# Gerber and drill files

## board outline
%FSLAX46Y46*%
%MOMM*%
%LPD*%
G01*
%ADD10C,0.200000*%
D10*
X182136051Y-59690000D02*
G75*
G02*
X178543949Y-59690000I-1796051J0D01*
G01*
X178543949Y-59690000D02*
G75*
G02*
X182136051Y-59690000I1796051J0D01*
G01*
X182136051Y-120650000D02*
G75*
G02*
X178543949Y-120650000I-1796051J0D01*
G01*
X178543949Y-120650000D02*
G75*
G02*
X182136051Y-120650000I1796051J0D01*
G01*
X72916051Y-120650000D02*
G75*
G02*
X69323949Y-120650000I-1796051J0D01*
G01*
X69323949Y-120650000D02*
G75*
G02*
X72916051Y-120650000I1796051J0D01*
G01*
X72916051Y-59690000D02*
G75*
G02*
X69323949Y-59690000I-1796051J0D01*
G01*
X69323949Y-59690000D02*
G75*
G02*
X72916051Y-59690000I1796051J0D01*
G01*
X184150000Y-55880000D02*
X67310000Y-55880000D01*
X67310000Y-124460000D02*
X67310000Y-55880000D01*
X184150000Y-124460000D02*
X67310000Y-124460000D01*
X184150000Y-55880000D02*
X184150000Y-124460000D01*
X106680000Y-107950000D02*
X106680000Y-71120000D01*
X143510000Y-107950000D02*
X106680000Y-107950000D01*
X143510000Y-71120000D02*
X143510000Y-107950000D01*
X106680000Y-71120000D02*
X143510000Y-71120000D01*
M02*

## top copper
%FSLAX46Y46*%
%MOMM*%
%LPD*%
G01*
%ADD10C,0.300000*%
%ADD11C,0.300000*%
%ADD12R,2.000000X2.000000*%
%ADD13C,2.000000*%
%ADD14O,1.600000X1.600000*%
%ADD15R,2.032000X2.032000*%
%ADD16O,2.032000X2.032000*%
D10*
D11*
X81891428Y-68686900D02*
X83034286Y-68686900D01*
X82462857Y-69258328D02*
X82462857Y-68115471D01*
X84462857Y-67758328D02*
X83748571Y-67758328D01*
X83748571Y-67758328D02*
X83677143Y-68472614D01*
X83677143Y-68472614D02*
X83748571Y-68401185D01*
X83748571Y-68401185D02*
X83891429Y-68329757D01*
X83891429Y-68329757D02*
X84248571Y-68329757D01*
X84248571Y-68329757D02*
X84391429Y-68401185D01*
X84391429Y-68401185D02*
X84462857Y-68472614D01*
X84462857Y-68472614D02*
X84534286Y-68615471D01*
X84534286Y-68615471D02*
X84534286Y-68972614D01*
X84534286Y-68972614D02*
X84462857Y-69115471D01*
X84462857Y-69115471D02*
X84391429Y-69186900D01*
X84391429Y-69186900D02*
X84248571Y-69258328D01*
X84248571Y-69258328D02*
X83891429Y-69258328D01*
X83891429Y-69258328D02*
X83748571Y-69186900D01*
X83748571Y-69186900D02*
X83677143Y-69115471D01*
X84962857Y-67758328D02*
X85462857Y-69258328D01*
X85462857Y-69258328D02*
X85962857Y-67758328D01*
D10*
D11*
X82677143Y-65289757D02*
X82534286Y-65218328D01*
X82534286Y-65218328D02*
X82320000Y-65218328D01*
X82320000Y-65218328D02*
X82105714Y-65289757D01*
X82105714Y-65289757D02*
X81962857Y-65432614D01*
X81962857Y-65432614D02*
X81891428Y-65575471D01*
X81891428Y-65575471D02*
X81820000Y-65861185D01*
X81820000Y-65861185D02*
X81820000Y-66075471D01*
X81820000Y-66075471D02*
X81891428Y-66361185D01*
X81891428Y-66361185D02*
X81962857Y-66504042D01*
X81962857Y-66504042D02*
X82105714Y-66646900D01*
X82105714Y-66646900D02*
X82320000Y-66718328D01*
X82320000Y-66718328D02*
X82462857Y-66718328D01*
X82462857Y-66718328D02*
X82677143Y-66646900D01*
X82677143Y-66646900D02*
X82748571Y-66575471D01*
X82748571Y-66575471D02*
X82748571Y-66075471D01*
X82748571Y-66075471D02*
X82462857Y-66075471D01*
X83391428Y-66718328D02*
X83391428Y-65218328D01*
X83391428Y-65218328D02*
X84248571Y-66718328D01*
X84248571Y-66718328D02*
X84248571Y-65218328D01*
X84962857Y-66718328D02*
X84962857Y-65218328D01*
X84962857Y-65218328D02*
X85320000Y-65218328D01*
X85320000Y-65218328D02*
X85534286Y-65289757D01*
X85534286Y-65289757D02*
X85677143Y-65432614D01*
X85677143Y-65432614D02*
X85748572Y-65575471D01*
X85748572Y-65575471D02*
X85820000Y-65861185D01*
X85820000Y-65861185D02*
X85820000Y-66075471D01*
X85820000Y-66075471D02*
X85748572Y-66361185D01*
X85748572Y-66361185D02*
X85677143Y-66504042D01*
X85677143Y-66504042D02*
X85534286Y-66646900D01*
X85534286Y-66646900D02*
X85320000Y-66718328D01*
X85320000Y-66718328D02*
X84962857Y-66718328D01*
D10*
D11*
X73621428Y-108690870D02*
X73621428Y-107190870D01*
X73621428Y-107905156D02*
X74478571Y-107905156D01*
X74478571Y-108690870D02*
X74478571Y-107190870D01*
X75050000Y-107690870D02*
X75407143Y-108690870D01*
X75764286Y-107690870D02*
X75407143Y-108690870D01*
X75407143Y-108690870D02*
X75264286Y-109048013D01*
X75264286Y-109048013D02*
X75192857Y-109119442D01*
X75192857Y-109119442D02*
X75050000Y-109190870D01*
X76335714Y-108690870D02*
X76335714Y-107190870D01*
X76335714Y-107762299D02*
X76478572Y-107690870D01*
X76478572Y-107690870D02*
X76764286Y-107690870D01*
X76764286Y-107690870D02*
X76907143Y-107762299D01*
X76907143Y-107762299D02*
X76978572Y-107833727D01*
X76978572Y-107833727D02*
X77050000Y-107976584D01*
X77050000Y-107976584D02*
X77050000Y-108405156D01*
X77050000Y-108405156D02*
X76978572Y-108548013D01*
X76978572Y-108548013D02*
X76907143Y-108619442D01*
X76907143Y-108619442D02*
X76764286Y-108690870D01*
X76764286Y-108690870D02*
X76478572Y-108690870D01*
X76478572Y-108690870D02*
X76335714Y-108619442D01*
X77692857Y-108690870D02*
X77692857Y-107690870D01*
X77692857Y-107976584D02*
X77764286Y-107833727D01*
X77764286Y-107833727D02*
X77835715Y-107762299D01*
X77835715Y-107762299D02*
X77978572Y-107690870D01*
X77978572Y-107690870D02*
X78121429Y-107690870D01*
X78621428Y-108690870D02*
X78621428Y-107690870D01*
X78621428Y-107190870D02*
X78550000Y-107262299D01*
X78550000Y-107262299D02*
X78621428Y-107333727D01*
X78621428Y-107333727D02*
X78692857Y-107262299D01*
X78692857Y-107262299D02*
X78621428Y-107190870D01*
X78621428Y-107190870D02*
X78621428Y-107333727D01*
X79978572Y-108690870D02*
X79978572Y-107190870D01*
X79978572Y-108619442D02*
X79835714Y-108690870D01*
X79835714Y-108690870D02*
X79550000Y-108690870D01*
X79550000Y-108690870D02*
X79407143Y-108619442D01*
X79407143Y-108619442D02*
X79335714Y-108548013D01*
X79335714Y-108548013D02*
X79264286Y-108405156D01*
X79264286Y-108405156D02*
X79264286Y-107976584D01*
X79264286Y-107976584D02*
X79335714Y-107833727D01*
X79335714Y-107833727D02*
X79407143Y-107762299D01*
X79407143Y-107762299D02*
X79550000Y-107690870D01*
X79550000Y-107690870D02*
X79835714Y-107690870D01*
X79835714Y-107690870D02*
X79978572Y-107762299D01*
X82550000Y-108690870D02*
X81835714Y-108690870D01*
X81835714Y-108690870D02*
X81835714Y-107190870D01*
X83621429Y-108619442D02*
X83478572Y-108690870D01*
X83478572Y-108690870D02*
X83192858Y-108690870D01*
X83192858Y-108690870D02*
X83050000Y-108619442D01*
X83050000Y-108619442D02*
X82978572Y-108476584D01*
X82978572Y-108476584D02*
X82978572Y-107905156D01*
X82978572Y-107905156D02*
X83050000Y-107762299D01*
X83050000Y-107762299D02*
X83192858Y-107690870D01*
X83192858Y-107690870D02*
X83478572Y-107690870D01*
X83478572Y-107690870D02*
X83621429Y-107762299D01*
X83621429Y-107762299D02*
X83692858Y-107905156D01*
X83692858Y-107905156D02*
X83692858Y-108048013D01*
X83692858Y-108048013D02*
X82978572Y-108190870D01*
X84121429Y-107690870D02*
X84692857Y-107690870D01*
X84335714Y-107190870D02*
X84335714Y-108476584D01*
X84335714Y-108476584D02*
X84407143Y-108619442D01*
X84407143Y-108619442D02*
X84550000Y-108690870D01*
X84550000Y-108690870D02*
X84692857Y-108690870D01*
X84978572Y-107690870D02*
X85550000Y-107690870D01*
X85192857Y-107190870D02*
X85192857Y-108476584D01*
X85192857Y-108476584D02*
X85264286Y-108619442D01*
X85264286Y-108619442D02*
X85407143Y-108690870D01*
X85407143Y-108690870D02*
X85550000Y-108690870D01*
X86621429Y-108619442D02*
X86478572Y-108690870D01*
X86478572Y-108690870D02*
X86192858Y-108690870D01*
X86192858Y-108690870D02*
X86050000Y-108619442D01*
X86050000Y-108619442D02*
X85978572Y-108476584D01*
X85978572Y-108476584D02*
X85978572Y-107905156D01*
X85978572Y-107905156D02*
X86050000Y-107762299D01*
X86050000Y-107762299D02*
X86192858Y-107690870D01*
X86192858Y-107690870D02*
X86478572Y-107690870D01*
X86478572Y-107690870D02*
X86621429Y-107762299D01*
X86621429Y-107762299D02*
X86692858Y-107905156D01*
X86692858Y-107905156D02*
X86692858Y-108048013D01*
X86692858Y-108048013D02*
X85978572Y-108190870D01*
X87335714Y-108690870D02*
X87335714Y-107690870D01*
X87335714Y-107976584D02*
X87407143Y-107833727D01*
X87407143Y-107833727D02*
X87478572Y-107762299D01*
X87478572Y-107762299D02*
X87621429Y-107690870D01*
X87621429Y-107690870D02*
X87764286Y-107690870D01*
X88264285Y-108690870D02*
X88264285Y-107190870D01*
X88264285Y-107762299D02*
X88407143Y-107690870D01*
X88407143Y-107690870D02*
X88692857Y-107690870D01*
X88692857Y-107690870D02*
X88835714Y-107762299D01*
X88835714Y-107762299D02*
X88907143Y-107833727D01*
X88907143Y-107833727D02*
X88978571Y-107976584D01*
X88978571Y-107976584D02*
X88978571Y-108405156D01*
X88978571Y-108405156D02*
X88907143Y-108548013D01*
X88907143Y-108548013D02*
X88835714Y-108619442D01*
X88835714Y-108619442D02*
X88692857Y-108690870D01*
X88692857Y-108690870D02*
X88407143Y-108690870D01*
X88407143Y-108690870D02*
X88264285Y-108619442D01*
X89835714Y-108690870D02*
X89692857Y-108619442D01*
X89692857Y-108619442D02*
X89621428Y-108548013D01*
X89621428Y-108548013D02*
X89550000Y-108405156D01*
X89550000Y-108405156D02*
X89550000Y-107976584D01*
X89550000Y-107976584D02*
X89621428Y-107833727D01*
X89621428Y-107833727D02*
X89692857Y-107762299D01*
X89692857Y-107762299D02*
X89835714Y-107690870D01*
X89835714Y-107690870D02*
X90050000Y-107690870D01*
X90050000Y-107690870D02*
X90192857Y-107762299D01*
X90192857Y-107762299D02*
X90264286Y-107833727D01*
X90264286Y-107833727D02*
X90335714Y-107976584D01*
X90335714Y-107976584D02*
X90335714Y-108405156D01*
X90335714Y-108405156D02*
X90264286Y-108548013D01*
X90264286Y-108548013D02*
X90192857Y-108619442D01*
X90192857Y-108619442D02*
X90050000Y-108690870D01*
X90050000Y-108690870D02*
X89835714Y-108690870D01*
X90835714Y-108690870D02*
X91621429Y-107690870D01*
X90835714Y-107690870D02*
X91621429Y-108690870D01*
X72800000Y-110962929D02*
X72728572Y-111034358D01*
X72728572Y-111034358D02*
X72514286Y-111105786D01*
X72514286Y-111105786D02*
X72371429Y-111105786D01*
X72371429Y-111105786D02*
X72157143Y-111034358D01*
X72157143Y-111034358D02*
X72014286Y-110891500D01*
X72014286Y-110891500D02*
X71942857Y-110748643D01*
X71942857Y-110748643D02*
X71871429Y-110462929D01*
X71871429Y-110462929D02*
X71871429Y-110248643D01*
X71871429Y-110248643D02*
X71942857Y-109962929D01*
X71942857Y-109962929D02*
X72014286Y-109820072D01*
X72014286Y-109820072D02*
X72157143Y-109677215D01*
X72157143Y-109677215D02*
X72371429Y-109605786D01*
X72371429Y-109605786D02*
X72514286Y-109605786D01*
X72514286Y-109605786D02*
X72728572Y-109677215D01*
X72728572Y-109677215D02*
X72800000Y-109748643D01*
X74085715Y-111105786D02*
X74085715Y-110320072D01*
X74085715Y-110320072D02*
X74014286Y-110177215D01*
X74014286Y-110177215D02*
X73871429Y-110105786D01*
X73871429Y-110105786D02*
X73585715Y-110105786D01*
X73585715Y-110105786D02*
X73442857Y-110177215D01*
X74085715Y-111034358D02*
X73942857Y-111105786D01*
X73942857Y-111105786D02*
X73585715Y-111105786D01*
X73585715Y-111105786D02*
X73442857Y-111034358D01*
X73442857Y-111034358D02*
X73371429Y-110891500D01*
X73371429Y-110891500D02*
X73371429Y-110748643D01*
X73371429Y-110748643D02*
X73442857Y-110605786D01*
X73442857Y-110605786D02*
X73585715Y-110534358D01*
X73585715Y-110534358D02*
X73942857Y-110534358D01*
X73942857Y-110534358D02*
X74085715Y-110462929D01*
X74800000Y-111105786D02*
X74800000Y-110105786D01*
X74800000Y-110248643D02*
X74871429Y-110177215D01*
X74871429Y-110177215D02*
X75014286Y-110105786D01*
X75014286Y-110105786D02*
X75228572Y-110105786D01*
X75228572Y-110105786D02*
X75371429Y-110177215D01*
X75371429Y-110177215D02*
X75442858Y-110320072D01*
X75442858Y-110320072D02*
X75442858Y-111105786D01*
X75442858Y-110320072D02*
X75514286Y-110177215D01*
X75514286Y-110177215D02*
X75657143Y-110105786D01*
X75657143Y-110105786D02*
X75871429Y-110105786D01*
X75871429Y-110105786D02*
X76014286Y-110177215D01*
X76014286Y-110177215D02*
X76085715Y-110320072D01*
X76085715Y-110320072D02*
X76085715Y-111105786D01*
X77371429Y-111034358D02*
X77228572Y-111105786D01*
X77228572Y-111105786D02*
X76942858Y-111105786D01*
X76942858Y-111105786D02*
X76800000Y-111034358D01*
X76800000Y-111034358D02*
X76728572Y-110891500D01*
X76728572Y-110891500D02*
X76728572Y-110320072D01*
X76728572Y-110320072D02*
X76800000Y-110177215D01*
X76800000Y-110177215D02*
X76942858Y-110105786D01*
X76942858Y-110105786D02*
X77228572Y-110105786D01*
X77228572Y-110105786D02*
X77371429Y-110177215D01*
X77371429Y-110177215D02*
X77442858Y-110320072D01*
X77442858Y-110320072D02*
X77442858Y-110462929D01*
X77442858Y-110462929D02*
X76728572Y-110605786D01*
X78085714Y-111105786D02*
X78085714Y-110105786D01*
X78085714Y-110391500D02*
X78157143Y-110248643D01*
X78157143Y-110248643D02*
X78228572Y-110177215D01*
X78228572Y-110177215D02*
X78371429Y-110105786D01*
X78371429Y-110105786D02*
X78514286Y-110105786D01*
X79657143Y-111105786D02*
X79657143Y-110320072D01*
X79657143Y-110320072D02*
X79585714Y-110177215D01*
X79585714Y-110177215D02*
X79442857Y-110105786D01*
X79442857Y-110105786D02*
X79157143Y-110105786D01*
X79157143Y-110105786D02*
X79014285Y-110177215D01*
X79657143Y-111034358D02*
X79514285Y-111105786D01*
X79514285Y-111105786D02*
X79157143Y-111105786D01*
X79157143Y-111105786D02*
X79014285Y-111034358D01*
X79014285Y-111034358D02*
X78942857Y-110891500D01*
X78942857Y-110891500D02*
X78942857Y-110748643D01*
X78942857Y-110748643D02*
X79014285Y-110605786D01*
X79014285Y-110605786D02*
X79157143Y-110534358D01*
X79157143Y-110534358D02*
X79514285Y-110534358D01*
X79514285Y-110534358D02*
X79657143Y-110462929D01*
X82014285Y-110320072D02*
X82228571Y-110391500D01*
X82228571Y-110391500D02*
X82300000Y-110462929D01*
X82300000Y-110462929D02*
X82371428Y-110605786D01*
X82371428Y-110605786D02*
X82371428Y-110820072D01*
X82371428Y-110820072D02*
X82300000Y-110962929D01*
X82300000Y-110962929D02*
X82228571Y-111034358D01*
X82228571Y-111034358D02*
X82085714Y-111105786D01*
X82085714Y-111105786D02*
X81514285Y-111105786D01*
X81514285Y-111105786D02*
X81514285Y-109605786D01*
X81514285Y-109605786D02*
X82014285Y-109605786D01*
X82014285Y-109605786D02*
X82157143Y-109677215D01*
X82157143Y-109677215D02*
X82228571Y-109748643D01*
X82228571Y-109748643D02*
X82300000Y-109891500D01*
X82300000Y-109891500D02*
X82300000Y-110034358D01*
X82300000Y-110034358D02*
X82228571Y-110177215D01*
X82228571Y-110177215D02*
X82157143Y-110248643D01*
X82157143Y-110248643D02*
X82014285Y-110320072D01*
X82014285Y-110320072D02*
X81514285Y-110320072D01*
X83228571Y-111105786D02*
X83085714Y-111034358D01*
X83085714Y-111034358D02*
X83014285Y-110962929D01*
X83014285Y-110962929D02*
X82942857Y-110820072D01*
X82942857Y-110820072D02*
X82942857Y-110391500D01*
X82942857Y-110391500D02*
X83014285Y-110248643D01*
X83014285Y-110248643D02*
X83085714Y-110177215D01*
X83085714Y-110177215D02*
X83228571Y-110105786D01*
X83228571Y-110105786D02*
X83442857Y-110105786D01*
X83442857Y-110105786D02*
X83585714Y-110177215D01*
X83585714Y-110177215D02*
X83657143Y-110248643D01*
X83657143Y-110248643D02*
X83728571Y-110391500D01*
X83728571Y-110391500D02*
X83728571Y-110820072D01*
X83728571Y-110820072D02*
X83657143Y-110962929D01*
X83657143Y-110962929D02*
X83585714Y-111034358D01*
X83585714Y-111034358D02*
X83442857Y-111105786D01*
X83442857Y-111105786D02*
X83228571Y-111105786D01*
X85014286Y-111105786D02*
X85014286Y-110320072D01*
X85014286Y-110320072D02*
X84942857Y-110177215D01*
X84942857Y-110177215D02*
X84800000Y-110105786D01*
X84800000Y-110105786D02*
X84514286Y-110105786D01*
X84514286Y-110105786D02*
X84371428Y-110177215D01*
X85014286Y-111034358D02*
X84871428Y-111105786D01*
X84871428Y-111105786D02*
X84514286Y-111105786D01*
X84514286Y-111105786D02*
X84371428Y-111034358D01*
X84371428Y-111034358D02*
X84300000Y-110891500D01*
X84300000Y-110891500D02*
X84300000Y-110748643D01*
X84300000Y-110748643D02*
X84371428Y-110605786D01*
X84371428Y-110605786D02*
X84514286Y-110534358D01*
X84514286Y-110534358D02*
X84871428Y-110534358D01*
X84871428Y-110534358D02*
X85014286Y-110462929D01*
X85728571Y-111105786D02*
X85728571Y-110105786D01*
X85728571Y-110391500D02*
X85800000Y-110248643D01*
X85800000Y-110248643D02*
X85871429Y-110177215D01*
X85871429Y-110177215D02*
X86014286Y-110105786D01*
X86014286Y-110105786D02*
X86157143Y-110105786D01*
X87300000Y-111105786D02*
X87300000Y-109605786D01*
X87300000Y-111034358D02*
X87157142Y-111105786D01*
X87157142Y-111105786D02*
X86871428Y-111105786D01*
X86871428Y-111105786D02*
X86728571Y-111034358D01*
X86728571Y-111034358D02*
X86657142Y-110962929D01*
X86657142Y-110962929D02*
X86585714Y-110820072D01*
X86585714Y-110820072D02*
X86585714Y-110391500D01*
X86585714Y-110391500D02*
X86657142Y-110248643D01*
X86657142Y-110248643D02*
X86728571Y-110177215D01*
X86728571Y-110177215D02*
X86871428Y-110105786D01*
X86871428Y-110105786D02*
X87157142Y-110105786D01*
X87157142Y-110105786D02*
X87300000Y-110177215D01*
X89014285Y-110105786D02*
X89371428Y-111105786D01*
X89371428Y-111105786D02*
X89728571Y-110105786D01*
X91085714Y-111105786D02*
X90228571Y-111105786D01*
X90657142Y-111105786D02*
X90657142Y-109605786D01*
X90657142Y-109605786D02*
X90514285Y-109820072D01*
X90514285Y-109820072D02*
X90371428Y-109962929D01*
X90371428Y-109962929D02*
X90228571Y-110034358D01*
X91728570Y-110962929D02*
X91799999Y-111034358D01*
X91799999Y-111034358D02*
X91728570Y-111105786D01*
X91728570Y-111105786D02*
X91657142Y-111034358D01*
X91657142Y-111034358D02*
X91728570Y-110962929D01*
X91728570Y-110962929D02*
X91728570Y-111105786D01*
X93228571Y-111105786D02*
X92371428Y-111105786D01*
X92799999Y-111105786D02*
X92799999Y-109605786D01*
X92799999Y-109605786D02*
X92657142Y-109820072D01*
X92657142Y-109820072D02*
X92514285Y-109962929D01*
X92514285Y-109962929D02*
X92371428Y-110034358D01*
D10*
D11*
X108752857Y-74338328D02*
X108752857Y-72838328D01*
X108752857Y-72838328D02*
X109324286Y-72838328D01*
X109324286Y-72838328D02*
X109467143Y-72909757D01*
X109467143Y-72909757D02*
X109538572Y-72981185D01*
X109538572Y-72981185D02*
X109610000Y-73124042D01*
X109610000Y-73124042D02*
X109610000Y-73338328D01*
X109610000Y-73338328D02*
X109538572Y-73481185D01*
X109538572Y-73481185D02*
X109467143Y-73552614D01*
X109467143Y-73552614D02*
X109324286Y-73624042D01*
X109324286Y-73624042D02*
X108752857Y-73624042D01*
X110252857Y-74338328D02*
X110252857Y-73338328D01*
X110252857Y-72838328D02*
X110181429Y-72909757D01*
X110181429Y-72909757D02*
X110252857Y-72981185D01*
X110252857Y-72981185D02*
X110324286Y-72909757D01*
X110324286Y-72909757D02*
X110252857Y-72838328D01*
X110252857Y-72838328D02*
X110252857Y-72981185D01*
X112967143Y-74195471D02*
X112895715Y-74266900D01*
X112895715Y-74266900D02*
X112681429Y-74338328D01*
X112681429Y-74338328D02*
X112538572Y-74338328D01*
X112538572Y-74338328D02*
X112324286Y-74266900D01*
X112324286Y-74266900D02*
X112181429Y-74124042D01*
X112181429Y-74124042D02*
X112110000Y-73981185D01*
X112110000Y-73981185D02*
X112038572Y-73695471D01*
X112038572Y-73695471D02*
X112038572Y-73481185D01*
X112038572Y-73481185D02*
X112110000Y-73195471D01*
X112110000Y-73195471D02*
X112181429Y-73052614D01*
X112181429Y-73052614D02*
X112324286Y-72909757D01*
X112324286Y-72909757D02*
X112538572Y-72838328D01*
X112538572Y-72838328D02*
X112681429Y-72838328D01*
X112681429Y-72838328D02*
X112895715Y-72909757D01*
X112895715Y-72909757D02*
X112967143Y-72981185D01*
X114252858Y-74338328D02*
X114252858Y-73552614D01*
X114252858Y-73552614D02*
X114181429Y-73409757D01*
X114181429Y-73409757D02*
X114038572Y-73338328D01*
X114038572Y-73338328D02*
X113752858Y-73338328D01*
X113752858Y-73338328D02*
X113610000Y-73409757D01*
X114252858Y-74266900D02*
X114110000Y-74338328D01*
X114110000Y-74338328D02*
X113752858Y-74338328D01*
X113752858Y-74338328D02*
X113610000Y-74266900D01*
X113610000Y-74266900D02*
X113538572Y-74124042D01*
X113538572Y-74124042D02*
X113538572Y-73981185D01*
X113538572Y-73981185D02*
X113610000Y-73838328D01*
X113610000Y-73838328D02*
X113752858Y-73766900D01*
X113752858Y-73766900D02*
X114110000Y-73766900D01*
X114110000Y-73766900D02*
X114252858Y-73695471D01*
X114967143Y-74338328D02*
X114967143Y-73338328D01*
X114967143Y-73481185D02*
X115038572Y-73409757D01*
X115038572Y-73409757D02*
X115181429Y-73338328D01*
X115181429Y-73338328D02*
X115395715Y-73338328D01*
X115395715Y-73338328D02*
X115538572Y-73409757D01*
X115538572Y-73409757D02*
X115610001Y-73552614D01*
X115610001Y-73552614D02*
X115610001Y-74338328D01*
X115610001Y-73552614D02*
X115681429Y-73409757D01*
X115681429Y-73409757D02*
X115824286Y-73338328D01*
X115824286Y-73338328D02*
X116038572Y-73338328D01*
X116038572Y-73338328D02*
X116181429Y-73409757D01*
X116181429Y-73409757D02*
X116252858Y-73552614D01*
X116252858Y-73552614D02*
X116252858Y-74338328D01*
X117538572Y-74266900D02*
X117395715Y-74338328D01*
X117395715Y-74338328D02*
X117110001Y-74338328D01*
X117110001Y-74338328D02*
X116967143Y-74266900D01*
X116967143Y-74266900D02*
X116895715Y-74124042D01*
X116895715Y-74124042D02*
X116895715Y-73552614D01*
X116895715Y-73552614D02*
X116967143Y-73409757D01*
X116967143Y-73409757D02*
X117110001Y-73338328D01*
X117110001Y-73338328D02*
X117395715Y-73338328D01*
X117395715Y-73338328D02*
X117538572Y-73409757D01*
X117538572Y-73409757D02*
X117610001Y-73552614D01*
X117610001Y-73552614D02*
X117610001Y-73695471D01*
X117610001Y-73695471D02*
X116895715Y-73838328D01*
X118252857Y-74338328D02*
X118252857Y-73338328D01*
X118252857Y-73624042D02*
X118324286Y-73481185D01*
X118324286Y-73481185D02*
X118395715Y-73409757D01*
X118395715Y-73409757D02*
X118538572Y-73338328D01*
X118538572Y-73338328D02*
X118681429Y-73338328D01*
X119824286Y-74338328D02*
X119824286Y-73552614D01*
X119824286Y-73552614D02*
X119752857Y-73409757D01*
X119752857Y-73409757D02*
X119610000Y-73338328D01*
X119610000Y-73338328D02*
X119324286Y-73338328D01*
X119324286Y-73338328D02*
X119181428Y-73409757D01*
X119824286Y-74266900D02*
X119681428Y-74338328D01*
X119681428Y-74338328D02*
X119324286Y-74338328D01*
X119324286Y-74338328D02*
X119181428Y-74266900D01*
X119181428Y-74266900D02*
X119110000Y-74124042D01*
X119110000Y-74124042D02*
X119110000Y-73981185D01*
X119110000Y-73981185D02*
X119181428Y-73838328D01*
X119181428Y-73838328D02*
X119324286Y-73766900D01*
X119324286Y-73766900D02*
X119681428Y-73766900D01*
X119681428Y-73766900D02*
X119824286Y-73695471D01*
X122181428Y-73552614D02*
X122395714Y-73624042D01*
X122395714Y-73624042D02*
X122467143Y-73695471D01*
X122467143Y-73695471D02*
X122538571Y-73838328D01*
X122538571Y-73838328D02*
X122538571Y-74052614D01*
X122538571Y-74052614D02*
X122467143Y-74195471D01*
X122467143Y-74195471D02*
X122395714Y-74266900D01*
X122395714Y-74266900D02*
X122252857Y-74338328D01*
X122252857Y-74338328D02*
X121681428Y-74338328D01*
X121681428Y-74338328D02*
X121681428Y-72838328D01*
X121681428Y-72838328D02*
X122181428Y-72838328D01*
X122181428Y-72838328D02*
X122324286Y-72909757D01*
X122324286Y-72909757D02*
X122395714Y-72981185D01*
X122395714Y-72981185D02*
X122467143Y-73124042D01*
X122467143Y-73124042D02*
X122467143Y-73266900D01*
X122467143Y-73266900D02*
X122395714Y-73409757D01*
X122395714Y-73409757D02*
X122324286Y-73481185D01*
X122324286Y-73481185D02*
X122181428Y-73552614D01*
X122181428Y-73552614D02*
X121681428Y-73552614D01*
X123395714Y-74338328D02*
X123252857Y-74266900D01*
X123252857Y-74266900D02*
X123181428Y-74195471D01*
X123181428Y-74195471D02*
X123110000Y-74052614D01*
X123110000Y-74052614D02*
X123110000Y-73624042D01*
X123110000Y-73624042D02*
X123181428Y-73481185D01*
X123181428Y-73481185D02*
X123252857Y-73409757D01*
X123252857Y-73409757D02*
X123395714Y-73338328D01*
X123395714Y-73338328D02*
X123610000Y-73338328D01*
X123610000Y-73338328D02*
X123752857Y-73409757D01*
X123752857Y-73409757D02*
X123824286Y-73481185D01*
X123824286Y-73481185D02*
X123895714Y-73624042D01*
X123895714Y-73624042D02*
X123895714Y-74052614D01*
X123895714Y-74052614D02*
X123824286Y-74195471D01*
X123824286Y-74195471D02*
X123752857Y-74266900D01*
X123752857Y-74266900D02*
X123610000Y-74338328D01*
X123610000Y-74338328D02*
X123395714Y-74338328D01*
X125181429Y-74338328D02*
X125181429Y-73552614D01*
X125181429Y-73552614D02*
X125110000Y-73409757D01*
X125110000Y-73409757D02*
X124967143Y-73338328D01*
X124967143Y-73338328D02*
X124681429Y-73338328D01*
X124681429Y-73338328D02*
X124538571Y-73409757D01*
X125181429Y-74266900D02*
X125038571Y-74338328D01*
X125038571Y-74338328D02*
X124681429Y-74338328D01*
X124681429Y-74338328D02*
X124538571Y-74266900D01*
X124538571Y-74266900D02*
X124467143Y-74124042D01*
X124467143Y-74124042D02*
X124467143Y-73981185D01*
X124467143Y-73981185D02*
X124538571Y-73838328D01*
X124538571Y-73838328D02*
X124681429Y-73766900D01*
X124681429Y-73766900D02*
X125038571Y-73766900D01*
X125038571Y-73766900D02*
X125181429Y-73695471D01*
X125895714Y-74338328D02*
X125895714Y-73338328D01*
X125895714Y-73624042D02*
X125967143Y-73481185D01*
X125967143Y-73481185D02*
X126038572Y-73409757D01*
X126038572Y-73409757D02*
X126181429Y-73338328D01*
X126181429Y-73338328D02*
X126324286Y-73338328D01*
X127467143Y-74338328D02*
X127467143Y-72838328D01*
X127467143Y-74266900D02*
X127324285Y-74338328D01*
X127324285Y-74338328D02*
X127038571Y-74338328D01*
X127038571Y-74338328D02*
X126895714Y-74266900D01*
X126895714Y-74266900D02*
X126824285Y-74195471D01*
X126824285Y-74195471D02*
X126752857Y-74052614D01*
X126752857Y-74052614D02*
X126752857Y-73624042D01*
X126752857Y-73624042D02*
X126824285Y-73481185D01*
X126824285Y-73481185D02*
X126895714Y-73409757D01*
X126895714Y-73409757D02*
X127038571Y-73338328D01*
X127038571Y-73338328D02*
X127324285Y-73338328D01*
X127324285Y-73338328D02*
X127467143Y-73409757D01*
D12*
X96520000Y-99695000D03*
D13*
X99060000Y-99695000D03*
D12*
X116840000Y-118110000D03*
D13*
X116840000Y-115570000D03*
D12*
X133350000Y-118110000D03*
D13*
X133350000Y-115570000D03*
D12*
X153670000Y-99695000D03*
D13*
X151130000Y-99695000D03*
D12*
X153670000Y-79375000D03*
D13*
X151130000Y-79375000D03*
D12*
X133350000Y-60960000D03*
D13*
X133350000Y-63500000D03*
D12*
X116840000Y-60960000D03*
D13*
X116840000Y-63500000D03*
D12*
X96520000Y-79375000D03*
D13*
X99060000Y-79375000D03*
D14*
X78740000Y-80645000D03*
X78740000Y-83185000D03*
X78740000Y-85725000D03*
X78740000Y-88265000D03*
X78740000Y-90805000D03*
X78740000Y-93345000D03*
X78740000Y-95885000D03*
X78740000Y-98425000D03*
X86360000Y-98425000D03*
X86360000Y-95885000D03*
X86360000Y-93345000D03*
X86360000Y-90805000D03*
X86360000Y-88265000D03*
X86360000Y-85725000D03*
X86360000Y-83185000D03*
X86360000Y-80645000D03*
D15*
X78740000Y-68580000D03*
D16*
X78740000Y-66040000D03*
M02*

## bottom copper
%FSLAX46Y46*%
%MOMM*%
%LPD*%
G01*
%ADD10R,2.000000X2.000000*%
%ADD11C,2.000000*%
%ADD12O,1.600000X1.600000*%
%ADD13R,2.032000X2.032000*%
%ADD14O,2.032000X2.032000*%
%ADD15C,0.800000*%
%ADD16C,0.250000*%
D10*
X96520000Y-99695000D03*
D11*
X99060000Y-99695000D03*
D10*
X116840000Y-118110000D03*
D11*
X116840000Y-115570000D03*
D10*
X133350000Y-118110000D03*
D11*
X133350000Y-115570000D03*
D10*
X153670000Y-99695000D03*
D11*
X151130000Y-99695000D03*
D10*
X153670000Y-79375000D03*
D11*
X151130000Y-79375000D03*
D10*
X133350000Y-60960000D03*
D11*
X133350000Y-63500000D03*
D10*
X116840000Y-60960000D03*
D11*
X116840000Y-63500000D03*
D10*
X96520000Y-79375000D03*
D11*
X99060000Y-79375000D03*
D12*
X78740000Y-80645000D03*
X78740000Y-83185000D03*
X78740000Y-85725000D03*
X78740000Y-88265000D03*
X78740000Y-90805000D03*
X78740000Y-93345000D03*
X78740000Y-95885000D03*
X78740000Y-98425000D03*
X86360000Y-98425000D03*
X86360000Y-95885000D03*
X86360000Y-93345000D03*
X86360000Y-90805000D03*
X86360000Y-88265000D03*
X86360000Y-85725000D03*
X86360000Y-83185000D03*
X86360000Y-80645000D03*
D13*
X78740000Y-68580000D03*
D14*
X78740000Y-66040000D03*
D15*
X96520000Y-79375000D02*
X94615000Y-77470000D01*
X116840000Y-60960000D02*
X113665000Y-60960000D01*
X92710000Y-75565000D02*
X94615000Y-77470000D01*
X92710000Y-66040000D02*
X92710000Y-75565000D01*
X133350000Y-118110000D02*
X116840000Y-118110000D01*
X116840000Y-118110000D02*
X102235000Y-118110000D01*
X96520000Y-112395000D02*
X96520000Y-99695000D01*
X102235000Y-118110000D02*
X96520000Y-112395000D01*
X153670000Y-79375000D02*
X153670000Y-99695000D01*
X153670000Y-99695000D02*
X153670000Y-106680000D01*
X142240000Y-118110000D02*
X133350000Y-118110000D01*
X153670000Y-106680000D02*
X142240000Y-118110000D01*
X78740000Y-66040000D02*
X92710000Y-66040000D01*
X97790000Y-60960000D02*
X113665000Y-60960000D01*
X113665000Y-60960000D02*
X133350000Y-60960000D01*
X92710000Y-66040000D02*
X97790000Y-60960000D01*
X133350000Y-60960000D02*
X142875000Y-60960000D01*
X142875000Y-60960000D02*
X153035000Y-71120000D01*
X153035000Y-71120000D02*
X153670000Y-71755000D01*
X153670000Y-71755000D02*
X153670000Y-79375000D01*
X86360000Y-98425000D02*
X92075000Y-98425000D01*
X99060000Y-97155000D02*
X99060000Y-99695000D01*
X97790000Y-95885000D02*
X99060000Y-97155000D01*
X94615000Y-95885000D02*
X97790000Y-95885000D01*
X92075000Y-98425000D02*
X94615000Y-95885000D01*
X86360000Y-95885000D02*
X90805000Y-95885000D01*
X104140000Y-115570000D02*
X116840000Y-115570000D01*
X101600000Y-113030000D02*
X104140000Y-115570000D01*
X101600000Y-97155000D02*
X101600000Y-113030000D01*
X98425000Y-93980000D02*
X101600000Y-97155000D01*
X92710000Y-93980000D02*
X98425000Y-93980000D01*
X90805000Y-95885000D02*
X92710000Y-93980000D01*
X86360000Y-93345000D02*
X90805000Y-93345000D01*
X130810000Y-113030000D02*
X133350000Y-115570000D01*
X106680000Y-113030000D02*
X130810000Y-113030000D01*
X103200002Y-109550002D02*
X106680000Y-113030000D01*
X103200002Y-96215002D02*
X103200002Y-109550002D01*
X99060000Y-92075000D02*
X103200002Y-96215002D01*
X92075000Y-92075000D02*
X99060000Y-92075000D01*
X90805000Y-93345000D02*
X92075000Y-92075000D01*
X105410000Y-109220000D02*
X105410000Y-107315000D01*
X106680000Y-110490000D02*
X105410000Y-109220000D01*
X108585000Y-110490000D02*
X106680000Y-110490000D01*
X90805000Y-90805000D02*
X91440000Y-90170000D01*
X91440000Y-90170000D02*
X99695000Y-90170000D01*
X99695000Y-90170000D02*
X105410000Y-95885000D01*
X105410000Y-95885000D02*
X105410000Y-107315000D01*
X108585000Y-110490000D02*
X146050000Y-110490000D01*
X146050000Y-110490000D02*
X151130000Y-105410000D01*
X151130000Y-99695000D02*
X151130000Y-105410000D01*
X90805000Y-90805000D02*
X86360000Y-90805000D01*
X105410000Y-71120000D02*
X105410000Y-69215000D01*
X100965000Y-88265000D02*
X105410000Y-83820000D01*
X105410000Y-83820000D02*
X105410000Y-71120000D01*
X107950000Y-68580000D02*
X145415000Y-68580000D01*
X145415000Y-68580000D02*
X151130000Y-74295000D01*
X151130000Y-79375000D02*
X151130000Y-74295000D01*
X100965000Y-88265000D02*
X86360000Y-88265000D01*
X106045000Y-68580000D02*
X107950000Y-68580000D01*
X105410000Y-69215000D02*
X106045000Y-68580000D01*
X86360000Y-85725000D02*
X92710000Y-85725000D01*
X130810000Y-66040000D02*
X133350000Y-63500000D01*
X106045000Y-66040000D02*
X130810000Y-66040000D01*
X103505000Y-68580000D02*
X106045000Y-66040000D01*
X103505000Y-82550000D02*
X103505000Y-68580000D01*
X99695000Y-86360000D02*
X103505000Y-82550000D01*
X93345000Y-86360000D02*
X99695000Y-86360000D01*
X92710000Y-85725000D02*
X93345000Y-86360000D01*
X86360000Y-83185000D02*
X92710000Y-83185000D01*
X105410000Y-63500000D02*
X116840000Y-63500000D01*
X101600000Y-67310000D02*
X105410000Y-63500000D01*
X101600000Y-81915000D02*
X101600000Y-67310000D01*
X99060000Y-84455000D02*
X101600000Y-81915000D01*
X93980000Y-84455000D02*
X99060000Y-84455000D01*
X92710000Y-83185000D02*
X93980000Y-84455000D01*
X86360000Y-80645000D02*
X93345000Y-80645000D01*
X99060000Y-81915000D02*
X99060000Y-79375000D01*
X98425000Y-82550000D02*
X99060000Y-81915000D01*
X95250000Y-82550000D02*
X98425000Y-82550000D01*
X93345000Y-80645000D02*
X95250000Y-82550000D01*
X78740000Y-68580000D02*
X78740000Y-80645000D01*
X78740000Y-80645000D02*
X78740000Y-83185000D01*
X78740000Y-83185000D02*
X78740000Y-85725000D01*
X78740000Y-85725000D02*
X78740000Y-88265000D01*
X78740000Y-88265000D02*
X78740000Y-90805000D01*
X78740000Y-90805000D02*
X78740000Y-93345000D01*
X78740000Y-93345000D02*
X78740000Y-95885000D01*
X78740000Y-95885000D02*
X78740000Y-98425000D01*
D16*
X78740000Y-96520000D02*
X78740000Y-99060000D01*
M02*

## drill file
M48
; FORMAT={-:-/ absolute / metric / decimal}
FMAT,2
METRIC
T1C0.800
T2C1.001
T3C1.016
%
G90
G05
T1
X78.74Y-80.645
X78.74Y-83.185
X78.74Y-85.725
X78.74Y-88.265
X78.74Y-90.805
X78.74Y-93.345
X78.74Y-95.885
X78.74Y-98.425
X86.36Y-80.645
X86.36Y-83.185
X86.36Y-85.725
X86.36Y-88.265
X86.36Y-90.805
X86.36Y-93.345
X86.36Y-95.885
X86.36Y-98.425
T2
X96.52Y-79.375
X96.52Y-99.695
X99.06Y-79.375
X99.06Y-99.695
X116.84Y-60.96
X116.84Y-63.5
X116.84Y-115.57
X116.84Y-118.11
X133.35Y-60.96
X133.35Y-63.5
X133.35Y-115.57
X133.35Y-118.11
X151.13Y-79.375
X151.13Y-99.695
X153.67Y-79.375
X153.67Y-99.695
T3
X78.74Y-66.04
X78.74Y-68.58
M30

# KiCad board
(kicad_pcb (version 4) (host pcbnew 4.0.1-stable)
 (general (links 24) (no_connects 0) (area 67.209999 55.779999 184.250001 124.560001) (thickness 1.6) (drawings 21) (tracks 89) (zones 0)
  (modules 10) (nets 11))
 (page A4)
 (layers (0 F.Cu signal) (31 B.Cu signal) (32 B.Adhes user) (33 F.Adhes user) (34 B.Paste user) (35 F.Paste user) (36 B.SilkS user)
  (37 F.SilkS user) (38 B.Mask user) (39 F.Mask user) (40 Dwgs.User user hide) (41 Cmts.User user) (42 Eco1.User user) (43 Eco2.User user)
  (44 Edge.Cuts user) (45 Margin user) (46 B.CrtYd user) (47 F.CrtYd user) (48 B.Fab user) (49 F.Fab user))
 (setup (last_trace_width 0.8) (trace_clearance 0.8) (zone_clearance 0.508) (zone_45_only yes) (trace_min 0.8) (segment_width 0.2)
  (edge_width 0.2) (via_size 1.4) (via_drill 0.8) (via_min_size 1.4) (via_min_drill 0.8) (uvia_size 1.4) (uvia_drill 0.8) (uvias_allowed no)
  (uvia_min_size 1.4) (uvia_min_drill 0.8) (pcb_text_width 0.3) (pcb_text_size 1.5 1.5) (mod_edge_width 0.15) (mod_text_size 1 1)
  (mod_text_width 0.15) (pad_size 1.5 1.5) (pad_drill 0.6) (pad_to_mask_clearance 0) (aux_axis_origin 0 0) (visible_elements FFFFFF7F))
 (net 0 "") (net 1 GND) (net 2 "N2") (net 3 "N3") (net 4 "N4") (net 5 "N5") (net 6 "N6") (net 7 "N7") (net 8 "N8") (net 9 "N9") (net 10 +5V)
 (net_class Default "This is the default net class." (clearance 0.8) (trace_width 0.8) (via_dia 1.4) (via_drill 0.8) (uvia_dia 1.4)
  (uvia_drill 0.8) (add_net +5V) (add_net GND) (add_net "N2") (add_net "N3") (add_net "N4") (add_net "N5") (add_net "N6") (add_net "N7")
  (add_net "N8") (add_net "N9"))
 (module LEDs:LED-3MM (layer F.Cu) (at 96.52 99.695)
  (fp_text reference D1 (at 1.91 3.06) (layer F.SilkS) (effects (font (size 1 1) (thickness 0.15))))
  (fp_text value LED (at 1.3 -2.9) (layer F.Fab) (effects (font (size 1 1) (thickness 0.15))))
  (pad 1 thru_hole rect (at 0 0 90) (size 2 2) (drill 1.00076) (layers *.Cu *.Mask F.SilkS) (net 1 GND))
  (pad 2 thru_hole circle (at 2.54 0) (size 2 2) (drill 1.00076) (layers *.Cu *.Mask F.SilkS) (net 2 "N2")))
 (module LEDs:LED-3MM (layer F.Cu) (at 116.84 118.11 90)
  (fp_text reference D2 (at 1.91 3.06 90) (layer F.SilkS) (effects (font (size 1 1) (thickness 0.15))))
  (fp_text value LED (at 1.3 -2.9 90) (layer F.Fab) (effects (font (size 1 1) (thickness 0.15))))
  (pad 1 thru_hole rect (at 0 0 180) (size 2 2) (drill 1.00076) (layers *.Cu *.Mask F.SilkS) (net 1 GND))
  (pad 2 thru_hole circle (at 2.54 0 90) (size 2 2) (drill 1.00076) (layers *.Cu *.Mask F.SilkS) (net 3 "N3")))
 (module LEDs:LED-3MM (layer F.Cu) (at 133.35 118.11 90)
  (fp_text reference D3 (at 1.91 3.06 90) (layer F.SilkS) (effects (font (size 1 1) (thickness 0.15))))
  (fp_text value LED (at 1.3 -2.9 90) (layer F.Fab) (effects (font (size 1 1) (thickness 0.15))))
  (pad 1 thru_hole rect (at 0 0 180) (size 2 2) (drill 1.00076) (layers *.Cu *.Mask F.SilkS) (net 1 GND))
  (pad 2 thru_hole circle (at 2.54 0 90) (size 2 2) (drill 1.00076) (layers *.Cu *.Mask F.SilkS) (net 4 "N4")))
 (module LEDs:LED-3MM (layer F.Cu) (at 153.67 99.695 180)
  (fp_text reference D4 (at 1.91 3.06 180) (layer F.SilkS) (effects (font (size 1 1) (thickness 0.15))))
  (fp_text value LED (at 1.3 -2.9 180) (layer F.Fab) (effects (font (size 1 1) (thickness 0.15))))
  (pad 1 thru_hole rect (at 0 0 270) (size 2 2) (drill 1.00076) (layers *.Cu *.Mask F.SilkS) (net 1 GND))
  (pad 2 thru_hole circle (at 2.54 0 180) (size 2 2) (drill 1.00076) (layers *.Cu *.Mask F.SilkS) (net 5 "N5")))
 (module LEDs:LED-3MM (layer F.Cu) (at 153.67 79.375 180)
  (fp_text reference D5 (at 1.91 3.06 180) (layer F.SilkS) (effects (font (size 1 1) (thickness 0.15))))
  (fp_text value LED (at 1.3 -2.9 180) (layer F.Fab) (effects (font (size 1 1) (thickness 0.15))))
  (pad 1 thru_hole rect (at 0 0 270) (size 2 2) (drill 1.00076) (layers *.Cu *.Mask F.SilkS) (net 1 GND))
  (pad 2 thru_hole circle (at 2.54 0 180) (size 2 2) (drill 1.00076) (layers *.Cu *.Mask F.SilkS) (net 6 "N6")))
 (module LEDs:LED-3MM (layer F.Cu) (at 133.35 60.96 270)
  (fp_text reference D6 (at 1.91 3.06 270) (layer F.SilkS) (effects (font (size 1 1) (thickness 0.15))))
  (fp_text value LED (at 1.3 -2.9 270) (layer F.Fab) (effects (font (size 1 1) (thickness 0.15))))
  (pad 1 thru_hole rect (at 0 0) (size 2 2) (drill 1.00076) (layers *.Cu *.Mask F.SilkS) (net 1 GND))
  (pad 2 thru_hole circle (at 2.54 0 270) (size 2 2) (drill 1.00076) (layers *.Cu *.Mask F.SilkS) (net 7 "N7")))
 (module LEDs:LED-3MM (layer F.Cu) (at 116.84 60.96 270)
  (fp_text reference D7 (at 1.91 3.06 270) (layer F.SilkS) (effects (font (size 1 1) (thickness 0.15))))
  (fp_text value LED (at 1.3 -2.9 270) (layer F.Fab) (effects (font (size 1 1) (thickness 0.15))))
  (pad 1 thru_hole rect (at 0 0) (size 2 2) (drill 1.00076) (layers *.Cu *.Mask F.SilkS) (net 1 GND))
  (pad 2 thru_hole circle (at 2.54 0 270) (size 2 2) (drill 1.00076) (layers *.Cu *.Mask F.SilkS) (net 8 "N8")))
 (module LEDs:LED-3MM (layer F.Cu) (at 96.52 79.375)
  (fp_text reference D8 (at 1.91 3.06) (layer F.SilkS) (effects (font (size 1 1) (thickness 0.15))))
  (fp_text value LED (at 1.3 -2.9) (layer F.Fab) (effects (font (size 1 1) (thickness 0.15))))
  (pad 1 thru_hole rect (at 0 0 90) (size 2 2) (drill 1.00076) (layers *.Cu *.Mask F.SilkS) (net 1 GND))
  (pad 2 thru_hole circle (at 2.54 0) (size 2 2) (drill 1.00076) (layers *.Cu *.Mask F.SilkS) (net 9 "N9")))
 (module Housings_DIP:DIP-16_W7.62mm (layer F.Cu) (at 78.74 80.645)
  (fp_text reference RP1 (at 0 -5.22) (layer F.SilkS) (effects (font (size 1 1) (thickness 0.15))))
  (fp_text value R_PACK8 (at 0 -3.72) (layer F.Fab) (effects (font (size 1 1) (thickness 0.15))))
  (pad 1 thru_hole oval (at 0 0) (size 1.6 1.6) (drill 0.8) (layers *.Cu *.Mask F.SilkS) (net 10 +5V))
  (pad 2 thru_hole oval (at 0 2.54) (size 1.6 1.6) (drill 0.8) (layers *.Cu *.Mask F.SilkS) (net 10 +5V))
  (pad 3 thru_hole oval (at 0 5.08) (size 1.6 1.6) (drill 0.8) (layers *.Cu *.Mask F.SilkS) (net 10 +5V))
  (pad 4 thru_hole oval (at 0 7.62) (size 1.6 1.6) (drill 0.8) (layers *.Cu *.Mask F.SilkS) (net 10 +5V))
  (pad 5 thru_hole oval (at 0 10.16) (size 1.6 1.6) (drill 0.8) (layers *.Cu *.Mask F.SilkS) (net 10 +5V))
  (pad 6 thru_hole oval (at 0 12.7) (size 1.6 1.6) (drill 0.8) (layers *.Cu *.Mask F.SilkS) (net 10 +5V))
  (pad 7 thru_hole oval (at 0 15.24) (size 1.6 1.6) (drill 0.8) (layers *.Cu *.Mask F.SilkS) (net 10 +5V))
  (pad 8 thru_hole oval (at 0 17.78) (size 1.6 1.6) (drill 0.8) (layers *.Cu *.Mask F.SilkS) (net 10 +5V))
  (pad 9 thru_hole oval (at 7.62 17.78) (size 1.6 1.6) (drill 0.8) (layers *.Cu *.Mask F.SilkS) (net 2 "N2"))
  (pad 10 thru_hole oval (at 7.62 15.24) (size 1.6 1.6) (drill 0.8) (layers *.Cu *.Mask F.SilkS) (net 3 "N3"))
  (pad 11 thru_hole oval (at 7.62 12.7) (size 1.6 1.6) (drill 0.8) (layers *.Cu *.Mask F.SilkS) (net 4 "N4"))
  (pad 12 thru_hole oval (at 7.62 10.16) (size 1.6 1.6) (drill 0.8) (layers *.Cu *.Mask F.SilkS) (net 5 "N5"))
  (pad 13 thru_hole oval (at 7.62 7.62) (size 1.6 1.6) (drill 0.8) (layers *.Cu *.Mask F.SilkS) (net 6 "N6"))
  (pad 14 thru_hole oval (at 7.62 5.08) (size 1.6 1.6) (drill 0.8) (layers *.Cu *.Mask F.SilkS) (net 7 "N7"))
  (pad 15 thru_hole oval (at 7.62 2.54) (size 1.6 1.6) (drill 0.8) (layers *.Cu *.Mask F.SilkS) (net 8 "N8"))
  (pad 16 thru_hole oval (at 7.62 0) (size 1.6 1.6) (drill 0.8) (layers *.Cu *.Mask F.SilkS) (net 9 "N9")))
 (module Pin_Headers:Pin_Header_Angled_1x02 (layer F.Cu) (at 78.74 68.58 180)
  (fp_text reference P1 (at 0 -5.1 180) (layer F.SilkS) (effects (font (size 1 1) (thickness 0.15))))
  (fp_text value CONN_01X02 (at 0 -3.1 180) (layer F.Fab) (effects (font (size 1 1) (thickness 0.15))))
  (pad 1 thru_hole rect (at 0 0 180) (size 2.032 2.032) (drill 1.016) (layers *.Cu *.Mask F.SilkS) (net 10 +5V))
  (pad 2 thru_hole oval (at 0 2.54 180) (size 2.032 2.032) (drill 1.016) (layers *.Cu *.Mask F.SilkS) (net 1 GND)))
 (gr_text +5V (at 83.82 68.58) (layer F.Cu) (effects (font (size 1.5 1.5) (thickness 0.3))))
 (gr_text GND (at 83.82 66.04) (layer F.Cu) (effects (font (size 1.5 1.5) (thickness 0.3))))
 (gr_circle (center 180.34 59.69) (end 179.07 60.96) (layer Edge.Cuts) (width 0.2))
 (gr_circle (center 180.34 120.65) (end 181.61 121.92) (layer Edge.Cuts) (width 0.2))
 (gr_circle (center 71.12 120.65) (end 72.39 119.38) (layer Edge.Cuts) (width 0.2))
 (gr_circle (center 71.12 59.69) (end 72.39 60.96) (layer Edge.Cuts) (width 0.2))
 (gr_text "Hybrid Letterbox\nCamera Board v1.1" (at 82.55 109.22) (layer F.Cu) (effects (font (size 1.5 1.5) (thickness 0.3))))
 (gr_line (start 184.15 55.88) (end 67.31 55.88) (angle 90) (layer Edge.Cuts) (width 0.2))
 (gr_line (start 67.31 124.46) (end 67.31 55.88) (angle 90) (layer Edge.Cuts) (width 0.2))
 (gr_line (start 184.15 124.46) (end 67.31 124.46) (angle 90) (layer Edge.Cuts) (width 0.2))
 (gr_line (start 184.15 55.88) (end 184.15 124.46) (angle 90) (layer Edge.Cuts) (width 0.2))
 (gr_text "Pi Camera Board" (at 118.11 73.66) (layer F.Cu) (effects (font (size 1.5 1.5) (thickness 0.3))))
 (gr_line (start 106.68 107.95) (end 106.68 71.12) (angle 90) (layer Edge.Cuts) (width 0.2))
 (gr_line (start 143.51 107.95) (end 106.68 107.95) (angle 90) (layer Edge.Cuts) (width 0.2))
 (gr_line (start 143.51 71.12) (end 143.51 107.95) (angle 90) (layer Edge.Cuts) (width 0.2))
 (gr_line (start 106.68 71.12) (end 143.51 71.12) (angle 90) (layer Edge.Cuts) (width 0.2))
 (segment (start 96.52 79.375) (end 94.615 77.47) (width 0.8) (layer B.Cu) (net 1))
 (segment (start 116.84 60.96) (end 113.665 60.96) (width 0.8) (layer B.Cu) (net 1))
 (segment (start 92.71 75.565) (end 94.615 77.47) (width 0.8) (layer B.Cu) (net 1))
 (segment (start 92.71 66.04) (end 92.71 75.565) (width 0.8) (layer B.Cu) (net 1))
 (segment (start 133.35 118.11) (end 116.84 118.11) (width 0.8) (layer B.Cu) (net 1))
 (segment (start 116.84 118.11) (end 102.235 118.11) (width 0.8) (layer B.Cu) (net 1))
 (segment (start 96.52 112.395) (end 96.52 99.695) (width 0.8) (layer B.Cu) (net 1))
 (segment (start 102.235 118.11) (end 96.52 112.395) (width 0.8) (layer B.Cu) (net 1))
 (segment (start 153.67 79.375) (end 153.67 99.695) (width 0.8) (layer B.Cu) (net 1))
 (segment (start 153.67 99.695) (end 153.67 106.68) (width 0.8) (layer B.Cu) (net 1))
 (segment (start 142.24 118.11) (end 133.35 118.11) (width 0.8) (layer B.Cu) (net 1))
 (segment (start 153.67 106.68) (end 142.24 118.11) (width 0.8) (layer B.Cu) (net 1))
 (segment (start 78.74 66.04) (end 92.71 66.04) (width 0.8) (layer B.Cu) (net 1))
 (segment (start 97.79 60.96) (end 113.665 60.96) (width 0.8) (layer B.Cu) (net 1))
 (segment (start 113.665 60.96) (end 133.35 60.96) (width 0.8) (layer B.Cu) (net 1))
 (segment (start 92.71 66.04) (end 97.79 60.96) (width 0.8) (layer B.Cu) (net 1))
 (segment (start 133.35 60.96) (end 142.875 60.96) (width 0.8) (layer B.Cu) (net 1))
 (segment (start 142.875 60.96) (end 153.035 71.12) (width 0.8) (layer B.Cu) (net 1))
 (segment (start 153.035 71.12) (end 153.67 71.755) (width 0.8) (layer B.Cu) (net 1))
 (segment (start 153.67 71.755) (end 153.67 79.375) (width 0.8) (layer B.Cu) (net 1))
 (segment (start 86.36 98.425) (end 92.075 98.425) (width 0.8) (layer B.Cu) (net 2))
 (segment (start 99.06 97.155) (end 99.06 99.695) (width 0.8) (layer B.Cu) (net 2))
 (segment (start 97.79 95.885) (end 99.06 97.155) (width 0.8) (layer B.Cu) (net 2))
 (segment (start 94.615 95.885) (end 97.79 95.885) (width 0.8) (layer B.Cu) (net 2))
 (segment (start 92.075 98.425) (end 94.615 95.885) (width 0.8) (layer B.Cu) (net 2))
 (segment (start 86.36 95.885) (end 90.805 95.885) (width 0.8) (layer B.Cu) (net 3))
 (segment (start 104.14 115.57) (end 116.84 115.57) (width 0.8) (layer B.Cu) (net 3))
 (segment (start 101.6 113.03) (end 104.14 115.57) (width 0.8) (layer B.Cu) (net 3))
 (segment (start 101.6 97.155) (end 101.6 113.03) (width 0.8) (layer B.Cu) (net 3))
 (segment (start 98.425 93.98) (end 101.6 97.155) (width 0.8) (layer B.Cu) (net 3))
 (segment (start 92.71 93.98) (end 98.425 93.98) (width 0.8) (layer B.Cu) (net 3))
 (segment (start 90.805 95.885) (end 92.71 93.98) (width 0.8) (layer B.Cu) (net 3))
 (segment (start 86.36 93.345) (end 90.805 93.345) (width 0.8) (layer B.Cu) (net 4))
 (segment (start 130.81 113.03) (end 133.35 115.57) (width 0.8) (layer B.Cu) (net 4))
 (segment (start 106.68 113.03) (end 130.81 113.03) (width 0.8) (layer B.Cu) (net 4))
 (segment (start 103.200002 109.550002) (end 106.68 113.03) (width 0.8) (layer B.Cu) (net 4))
 (segment (start 103.200002 96.215002) (end 103.200002 109.550002) (width 0.8) (layer B.Cu) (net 4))
 (segment (start 99.06 92.075) (end 103.200002 96.215002) (width 0.8) (layer B.Cu) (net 4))
 (segment (start 92.075 92.075) (end 99.06 92.075) (width 0.8) (layer B.Cu) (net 4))
 (segment (start 90.805 93.345) (end 92.075 92.075) (width 0.8) (layer B.Cu) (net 4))
 (segment (start 105.41 109.22) (end 105.41 107.315) (width 0.8) (layer B.Cu) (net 5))
 (segment (start 106.68 110.49) (end 105.41 109.22) (width 0.8) (layer B.Cu) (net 5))
 (segment (start 108.585 110.49) (end 106.68 110.49) (width 0.8) (layer B.Cu) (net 5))
 (segment (start 90.805 90.805) (end 91.44 90.17) (width 0.8) (layer B.Cu) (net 5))
 (segment (start 91.44 90.17) (end 99.695 90.17) (width 0.8) (layer B.Cu) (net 5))
 (segment (start 99.695 90.17) (end 105.41 95.885) (width 0.8) (layer B.Cu) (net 5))
 (segment (start 105.41 95.885) (end 105.41 107.315) (width 0.8) (layer B.Cu) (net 5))
 (segment (start 108.585 110.49) (end 146.05 110.49) (width 0.8) (layer B.Cu) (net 5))
 (segment (start 146.05 110.49) (end 151.13 105.41) (width 0.8) (layer B.Cu) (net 5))
 (segment (start 151.13 99.695) (end 151.13 105.41) (width 0.8) (layer B.Cu) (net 5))
 (segment (start 90.805 90.805) (end 86.36 90.805) (width 0.8) (layer B.Cu) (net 5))
 (segment (start 105.41 71.12) (end 105.41 69.215) (width 0.8) (layer B.Cu) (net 6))
 (segment (start 100.965 88.265) (end 105.41 83.82) (width 0.8) (layer B.Cu) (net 6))
 (segment (start 105.41 83.82) (end 105.41 71.12) (width 0.8) (layer B.Cu) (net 6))
 (segment (start 107.95 68.58) (end 145.415 68.58) (width 0.8) (layer B.Cu) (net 6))
 (segment (start 145.415 68.58) (end 151.13 74.295) (width 0.8) (layer B.Cu) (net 6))
 (segment (start 151.13 79.375) (end 151.13 74.295) (width 0.8) (layer B.Cu) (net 6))
 (segment (start 100.965 88.265) (end 86.36 88.265) (width 0.8) (layer B.Cu) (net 6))
 (segment (start 106.045 68.58) (end 107.95 68.58) (width 0.8) (layer B.Cu) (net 6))
 (segment (start 105.41 69.215) (end 106.045 68.58) (width 0.8) (layer B.Cu) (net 6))
 (segment (start 86.36 85.725) (end 92.71 85.725) (width 0.8) (layer B.Cu) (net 7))
 (segment (start 130.81 66.04) (end 133.35 63.5) (width 0.8) (layer B.Cu) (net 7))
 (segment (start 106.045 66.04) (end 130.81 66.04) (width 0.8) (layer B.Cu) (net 7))
 (segment (start 103.505 68.58) (end 106.045 66.04) (width 0.8) (layer B.Cu) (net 7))
 (segment (start 103.505 82.55) (end 103.505 68.58) (width 0.8) (layer B.Cu) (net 7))
 (segment (start 99.695 86.36) (end 103.505 82.55) (width 0.8) (layer B.Cu) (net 7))
 (segment (start 93.345 86.36) (end 99.695 86.36) (width 0.8) (layer B.Cu) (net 7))
 (segment (start 92.71 85.725) (end 93.345 86.36) (width 0.8) (layer B.Cu) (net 7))
 (segment (start 86.36 83.185) (end 92.71 83.185) (width 0.8) (layer B.Cu) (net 8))
 (segment (start 105.41 63.5) (end 116.84 63.5) (width 0.8) (layer B.Cu) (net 8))
 (segment (start 101.6 67.31) (end 105.41 63.5) (width 0.8) (layer B.Cu) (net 8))
 (segment (start 101.6 81.915) (end 101.6 67.31) (width 0.8) (layer B.Cu) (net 8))
 (segment (start 99.06 84.455) (end 101.6 81.915) (width 0.8) (layer B.Cu) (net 8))
 (segment (start 93.98 84.455) (end 99.06 84.455) (width 0.8) (layer B.Cu) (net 8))
 (segment (start 92.71 83.185) (end 93.98 84.455) (width 0.8) (layer B.Cu) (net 8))
 (segment (start 86.36 80.645) (end 93.345 80.645) (width 0.8) (layer B.Cu) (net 9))
 (segment (start 99.06 81.915) (end 99.06 79.375) (width 0.8) (layer B.Cu) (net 9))
 (segment (start 98.425 82.55) (end 99.06 81.915) (width 0.8) (layer B.Cu) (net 9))
 (segment (start 95.25 82.55) (end 98.425 82.55) (width 0.8) (layer B.Cu) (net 9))
 (segment (start 93.345 80.645) (end 95.25 82.55) (width 0.8) (layer B.Cu) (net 9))
 (segment (start 78.74 68.58) (end 78.74 80.645) (width 0.8) (layer B.Cu) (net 10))
 (segment (start 78.74 80.645) (end 78.74 83.185) (width 0.8) (layer B.Cu) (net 10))
 (segment (start 78.74 83.185) (end 78.74 85.725) (width 0.8) (layer B.Cu) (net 10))
 (segment (start 78.74 85.725) (end 78.74 88.265) (width 0.8) (layer B.Cu) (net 10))
 (segment (start 78.74 88.265) (end 78.74 90.805) (width 0.8) (layer B.Cu) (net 10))
 (segment (start 78.74 90.805) (end 78.74 93.345) (width 0.8) (layer B.Cu) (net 10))
 (segment (start 78.74 93.345) (end 78.74 95.885) (width 0.8) (layer B.Cu) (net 10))
 (segment (start 78.74 95.885) (end 78.74 98.425) (width 0.8) (layer B.Cu) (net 10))
 (segment (start 78.74 96.52) (end 78.74 99.06) (width 0.25) (layer B.Cu) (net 10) (status 30)))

